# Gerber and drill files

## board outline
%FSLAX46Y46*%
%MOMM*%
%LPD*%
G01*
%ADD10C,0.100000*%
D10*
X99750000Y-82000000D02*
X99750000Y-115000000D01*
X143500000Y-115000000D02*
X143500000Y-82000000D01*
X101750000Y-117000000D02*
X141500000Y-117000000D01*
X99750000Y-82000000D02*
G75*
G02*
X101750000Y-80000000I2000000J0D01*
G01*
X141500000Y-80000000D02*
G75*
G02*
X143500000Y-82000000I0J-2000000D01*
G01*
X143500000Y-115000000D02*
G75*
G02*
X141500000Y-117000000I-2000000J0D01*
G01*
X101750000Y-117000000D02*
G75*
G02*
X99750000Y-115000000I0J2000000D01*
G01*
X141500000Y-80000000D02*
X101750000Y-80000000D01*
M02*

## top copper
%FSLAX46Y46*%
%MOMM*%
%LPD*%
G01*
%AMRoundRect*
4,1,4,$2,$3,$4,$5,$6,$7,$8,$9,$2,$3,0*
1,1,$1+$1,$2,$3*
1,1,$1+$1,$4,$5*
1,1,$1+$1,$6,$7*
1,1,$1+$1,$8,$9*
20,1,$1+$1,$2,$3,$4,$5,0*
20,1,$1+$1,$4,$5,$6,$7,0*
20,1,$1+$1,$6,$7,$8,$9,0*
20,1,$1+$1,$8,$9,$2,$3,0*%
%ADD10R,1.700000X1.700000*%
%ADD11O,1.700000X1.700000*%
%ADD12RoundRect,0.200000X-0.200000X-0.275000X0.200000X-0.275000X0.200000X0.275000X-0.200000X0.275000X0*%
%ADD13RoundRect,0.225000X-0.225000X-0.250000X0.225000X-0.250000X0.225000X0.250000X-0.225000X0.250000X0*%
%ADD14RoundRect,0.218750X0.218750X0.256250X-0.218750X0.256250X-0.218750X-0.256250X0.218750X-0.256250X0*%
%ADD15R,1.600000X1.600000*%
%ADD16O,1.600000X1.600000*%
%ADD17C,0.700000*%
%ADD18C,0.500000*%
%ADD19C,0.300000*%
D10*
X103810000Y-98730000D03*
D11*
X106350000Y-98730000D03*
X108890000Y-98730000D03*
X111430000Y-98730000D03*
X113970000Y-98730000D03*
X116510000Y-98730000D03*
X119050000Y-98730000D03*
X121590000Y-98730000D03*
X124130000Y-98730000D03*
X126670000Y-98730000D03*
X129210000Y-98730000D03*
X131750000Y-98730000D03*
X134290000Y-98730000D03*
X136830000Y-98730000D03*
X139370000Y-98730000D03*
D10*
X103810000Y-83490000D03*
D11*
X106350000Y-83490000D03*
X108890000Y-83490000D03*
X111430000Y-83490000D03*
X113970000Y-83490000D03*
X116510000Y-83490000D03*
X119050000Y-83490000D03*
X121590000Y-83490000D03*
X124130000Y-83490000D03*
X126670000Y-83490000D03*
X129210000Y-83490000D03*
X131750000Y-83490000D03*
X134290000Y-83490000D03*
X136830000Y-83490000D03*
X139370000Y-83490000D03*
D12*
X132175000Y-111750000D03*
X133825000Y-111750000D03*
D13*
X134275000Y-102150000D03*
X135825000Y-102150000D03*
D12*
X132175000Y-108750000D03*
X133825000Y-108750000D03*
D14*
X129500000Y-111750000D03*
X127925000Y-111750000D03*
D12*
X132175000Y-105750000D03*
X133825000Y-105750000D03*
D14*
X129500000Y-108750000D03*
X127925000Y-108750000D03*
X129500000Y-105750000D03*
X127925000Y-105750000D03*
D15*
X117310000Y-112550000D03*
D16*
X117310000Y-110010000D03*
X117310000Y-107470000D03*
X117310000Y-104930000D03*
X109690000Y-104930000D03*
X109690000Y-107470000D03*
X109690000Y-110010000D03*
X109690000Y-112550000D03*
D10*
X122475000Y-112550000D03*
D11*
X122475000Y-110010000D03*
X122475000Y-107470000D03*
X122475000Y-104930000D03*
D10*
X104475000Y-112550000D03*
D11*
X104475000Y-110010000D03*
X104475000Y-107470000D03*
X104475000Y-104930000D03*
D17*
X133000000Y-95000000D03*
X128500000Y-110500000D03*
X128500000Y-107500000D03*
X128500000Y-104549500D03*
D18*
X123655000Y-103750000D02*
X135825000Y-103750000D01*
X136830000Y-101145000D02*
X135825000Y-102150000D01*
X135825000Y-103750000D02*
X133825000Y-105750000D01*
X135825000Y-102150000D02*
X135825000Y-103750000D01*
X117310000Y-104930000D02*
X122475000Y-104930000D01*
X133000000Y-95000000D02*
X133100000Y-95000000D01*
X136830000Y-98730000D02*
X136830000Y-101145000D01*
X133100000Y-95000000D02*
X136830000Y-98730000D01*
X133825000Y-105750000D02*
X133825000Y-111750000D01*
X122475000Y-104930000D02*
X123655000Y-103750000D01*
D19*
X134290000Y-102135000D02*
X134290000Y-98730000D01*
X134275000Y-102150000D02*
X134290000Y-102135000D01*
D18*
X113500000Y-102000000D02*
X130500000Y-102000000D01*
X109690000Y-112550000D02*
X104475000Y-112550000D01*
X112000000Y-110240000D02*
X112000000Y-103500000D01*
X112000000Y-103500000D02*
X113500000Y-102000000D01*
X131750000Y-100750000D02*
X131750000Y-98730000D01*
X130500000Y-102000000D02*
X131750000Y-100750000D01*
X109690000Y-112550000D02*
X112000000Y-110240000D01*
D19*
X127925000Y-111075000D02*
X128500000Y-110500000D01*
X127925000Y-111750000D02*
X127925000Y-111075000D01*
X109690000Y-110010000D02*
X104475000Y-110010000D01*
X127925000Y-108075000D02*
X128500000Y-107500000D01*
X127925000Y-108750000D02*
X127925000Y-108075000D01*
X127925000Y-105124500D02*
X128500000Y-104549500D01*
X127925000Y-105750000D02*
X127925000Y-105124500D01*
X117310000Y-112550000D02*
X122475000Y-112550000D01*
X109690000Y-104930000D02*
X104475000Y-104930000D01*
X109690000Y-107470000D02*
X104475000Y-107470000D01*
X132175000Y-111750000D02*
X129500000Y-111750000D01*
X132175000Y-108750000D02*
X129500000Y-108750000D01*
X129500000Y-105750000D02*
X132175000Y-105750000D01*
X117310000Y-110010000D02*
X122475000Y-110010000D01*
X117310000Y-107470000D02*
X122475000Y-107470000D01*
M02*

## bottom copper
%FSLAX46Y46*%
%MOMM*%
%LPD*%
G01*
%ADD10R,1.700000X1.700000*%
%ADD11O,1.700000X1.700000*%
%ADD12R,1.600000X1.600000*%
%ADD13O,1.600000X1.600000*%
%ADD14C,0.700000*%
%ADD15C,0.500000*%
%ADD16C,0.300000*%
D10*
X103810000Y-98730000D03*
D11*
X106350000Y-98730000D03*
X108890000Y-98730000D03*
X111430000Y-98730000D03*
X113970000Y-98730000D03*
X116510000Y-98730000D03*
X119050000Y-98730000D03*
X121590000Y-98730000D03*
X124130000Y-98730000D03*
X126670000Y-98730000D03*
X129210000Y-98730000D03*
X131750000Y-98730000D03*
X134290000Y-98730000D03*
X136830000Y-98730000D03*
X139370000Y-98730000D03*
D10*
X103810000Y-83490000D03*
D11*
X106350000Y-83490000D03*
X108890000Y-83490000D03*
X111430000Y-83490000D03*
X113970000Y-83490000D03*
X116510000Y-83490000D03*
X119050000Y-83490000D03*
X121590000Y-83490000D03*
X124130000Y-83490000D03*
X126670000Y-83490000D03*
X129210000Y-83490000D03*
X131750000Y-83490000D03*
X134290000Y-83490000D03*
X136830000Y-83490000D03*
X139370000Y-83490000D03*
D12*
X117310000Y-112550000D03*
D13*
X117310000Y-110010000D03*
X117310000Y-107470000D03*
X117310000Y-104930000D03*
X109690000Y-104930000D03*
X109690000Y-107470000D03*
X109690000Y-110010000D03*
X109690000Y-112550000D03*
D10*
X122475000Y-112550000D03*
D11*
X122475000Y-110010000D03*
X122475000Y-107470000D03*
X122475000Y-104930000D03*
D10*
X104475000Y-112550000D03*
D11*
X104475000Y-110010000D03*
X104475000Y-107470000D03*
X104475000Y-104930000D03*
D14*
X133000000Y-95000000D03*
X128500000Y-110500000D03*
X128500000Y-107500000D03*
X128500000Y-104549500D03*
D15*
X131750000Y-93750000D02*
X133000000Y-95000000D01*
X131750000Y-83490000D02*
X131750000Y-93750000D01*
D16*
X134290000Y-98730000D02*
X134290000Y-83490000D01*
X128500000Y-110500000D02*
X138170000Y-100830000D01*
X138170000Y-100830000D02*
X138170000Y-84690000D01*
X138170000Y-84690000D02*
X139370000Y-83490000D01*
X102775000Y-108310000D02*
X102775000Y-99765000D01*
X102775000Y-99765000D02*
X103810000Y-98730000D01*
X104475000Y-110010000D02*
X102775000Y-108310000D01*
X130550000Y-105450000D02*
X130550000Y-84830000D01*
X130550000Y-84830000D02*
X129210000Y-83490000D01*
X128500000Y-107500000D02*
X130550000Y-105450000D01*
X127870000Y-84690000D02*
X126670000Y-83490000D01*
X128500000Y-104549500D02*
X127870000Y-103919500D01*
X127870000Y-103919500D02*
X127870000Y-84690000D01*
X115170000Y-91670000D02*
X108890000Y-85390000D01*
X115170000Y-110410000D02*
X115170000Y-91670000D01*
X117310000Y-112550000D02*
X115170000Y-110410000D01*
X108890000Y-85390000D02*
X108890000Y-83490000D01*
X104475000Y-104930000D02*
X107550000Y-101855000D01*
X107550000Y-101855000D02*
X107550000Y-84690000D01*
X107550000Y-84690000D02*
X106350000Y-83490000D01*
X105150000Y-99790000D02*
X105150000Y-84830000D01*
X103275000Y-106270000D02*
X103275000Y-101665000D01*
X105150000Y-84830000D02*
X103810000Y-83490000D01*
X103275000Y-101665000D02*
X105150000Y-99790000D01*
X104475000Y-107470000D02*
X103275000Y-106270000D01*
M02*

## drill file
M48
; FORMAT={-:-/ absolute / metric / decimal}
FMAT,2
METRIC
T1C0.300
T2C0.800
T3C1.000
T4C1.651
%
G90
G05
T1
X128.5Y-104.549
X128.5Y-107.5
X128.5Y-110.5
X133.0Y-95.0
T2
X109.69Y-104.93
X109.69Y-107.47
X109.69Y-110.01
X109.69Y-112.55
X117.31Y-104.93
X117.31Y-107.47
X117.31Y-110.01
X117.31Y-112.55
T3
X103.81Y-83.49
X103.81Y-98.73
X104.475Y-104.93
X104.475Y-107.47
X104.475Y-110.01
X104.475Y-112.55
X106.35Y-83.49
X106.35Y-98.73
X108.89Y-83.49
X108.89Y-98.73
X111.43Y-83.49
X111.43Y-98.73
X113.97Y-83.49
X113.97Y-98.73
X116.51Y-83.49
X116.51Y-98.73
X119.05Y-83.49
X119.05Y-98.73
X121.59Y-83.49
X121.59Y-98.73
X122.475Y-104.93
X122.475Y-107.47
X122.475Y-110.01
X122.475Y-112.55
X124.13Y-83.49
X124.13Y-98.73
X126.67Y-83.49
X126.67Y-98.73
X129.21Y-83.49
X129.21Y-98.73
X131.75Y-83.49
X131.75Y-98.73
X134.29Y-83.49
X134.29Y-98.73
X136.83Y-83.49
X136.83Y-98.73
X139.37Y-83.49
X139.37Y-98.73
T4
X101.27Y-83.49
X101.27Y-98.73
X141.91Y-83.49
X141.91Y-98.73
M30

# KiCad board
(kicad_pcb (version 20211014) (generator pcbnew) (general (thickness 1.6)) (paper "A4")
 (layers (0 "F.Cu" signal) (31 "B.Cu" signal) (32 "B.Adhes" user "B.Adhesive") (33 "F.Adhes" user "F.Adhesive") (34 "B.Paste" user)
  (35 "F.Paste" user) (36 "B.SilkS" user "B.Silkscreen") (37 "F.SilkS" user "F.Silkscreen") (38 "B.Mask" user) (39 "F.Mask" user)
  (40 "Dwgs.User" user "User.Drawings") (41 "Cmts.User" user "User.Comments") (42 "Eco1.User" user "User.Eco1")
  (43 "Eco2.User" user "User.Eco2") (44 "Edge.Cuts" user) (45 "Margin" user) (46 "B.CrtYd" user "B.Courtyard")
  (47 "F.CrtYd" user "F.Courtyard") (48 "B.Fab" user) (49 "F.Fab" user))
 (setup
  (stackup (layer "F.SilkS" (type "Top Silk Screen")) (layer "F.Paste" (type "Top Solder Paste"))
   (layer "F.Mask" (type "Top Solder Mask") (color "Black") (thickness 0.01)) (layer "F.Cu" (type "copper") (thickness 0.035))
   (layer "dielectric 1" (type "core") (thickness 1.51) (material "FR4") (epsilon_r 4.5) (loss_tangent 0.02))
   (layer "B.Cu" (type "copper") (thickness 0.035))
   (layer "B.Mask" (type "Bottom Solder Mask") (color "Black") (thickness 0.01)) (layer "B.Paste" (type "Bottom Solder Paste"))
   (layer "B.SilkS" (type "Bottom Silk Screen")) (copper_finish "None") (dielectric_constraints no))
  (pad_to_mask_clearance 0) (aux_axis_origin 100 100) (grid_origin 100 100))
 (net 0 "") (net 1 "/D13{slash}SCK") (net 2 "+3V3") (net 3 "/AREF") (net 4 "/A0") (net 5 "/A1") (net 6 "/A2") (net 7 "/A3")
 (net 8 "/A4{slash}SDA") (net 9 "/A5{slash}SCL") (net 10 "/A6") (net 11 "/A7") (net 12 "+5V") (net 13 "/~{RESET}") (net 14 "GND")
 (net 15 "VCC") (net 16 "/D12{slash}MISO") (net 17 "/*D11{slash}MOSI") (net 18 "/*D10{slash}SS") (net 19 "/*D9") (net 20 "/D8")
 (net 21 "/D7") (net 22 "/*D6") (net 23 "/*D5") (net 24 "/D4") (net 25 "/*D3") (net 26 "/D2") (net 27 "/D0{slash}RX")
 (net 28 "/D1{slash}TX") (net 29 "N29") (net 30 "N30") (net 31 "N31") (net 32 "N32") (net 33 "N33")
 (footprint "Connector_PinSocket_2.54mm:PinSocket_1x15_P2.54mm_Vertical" (layer "F.Cu") (at 103.81 98.73 90)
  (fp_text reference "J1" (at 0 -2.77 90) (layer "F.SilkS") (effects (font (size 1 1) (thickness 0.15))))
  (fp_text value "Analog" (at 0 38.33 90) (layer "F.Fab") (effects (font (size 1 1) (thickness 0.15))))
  (pad "1" thru_hole rect (at 0 0 90) (size 1.7 1.7) (drill 1) (layers *.Cu *.Mask) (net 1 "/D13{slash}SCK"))
  (pad "2" thru_hole oval (at 0 2.54 90) (size 1.7 1.7) (drill 1) (layers *.Cu *.Mask) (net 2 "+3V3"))
  (pad "3" thru_hole oval (at 0 5.08 90) (size 1.7 1.7) (drill 1) (layers *.Cu *.Mask) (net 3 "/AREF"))
  (pad "4" thru_hole oval (at 0 7.62 90) (size 1.7 1.7) (drill 1) (layers *.Cu *.Mask) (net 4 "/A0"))
  (pad "5" thru_hole oval (at 0 10.16 90) (size 1.7 1.7) (drill 1) (layers *.Cu *.Mask) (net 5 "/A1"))
  (pad "6" thru_hole oval (at 0 12.7 90) (size 1.7 1.7) (drill 1) (layers *.Cu *.Mask) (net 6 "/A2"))
  (pad "7" thru_hole oval (at 0 15.24 90) (size 1.7 1.7) (drill 1) (layers *.Cu *.Mask) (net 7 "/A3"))
  (pad "8" thru_hole oval (at 0 17.78 90) (size 1.7 1.7) (drill 1) (layers *.Cu *.Mask) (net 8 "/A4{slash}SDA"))
  (pad "9" thru_hole oval (at 0 20.32 90) (size 1.7 1.7) (drill 1) (layers *.Cu *.Mask) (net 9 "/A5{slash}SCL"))
  (pad "10" thru_hole oval (at 0 22.86 90) (size 1.7 1.7) (drill 1) (layers *.Cu *.Mask) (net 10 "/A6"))
  (pad "11" thru_hole oval (at 0 25.4 90) (size 1.7 1.7) (drill 1) (layers *.Cu *.Mask) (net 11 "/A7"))
  (pad "12" thru_hole oval (at 0 27.94 90) (size 1.7 1.7) (drill 1) (layers *.Cu *.Mask) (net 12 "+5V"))
  (pad "13" thru_hole oval (at 0 30.48 90) (size 1.7 1.7) (drill 1) (layers *.Cu *.Mask) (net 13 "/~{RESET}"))
  (pad "14" thru_hole oval (at 0 33.02 90) (size 1.7 1.7) (drill 1) (layers *.Cu *.Mask) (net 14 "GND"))
  (pad "15" thru_hole oval (at 0 35.56 90) (size 1.7 1.7) (drill 1) (layers *.Cu *.Mask) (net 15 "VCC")))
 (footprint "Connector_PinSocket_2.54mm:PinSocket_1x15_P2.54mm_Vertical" (layer "F.Cu") (at 103.81 83.49 90)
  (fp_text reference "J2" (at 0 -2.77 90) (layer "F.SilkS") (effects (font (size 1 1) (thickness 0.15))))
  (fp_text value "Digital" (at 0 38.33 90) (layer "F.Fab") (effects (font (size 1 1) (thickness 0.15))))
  (pad "1" thru_hole rect (at 0 0 90) (size 1.7 1.7) (drill 1) (layers *.Cu *.Mask) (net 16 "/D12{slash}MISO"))
  (pad "2" thru_hole oval (at 0 2.54 90) (size 1.7 1.7) (drill 1) (layers *.Cu *.Mask) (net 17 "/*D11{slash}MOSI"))
  (pad "3" thru_hole oval (at 0 5.08 90) (size 1.7 1.7) (drill 1) (layers *.Cu *.Mask) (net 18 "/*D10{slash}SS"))
  (pad "4" thru_hole oval (at 0 7.62 90) (size 1.7 1.7) (drill 1) (layers *.Cu *.Mask) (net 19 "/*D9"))
  (pad "5" thru_hole oval (at 0 10.16 90) (size 1.7 1.7) (drill 1) (layers *.Cu *.Mask) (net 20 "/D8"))
  (pad "6" thru_hole oval (at 0 12.7 90) (size 1.7 1.7) (drill 1) (layers *.Cu *.Mask) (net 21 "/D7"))
  (pad "7" thru_hole oval (at 0 15.24 90) (size 1.7 1.7) (drill 1) (layers *.Cu *.Mask) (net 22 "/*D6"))
  (pad "8" thru_hole oval (at 0 17.78 90) (size 1.7 1.7) (drill 1) (layers *.Cu *.Mask) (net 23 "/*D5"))
  (pad "9" thru_hole oval (at 0 20.32 90) (size 1.7 1.7) (drill 1) (layers *.Cu *.Mask) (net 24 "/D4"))
  (pad "10" thru_hole oval (at 0 22.86 90) (size 1.7 1.7) (drill 1) (layers *.Cu *.Mask) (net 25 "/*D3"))
  (pad "11" thru_hole oval (at 0 25.4 90) (size 1.7 1.7) (drill 1) (layers *.Cu *.Mask) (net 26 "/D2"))
  (pad "12" thru_hole oval (at 0 27.94 90) (size 1.7 1.7) (drill 1) (layers *.Cu *.Mask) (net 14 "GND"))
  (pad "13" thru_hole oval (at 0 30.48 90) (size 1.7 1.7) (drill 1) (layers *.Cu *.Mask) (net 13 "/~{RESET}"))
  (pad "14" thru_hole oval (at 0 33.02 90) (size 1.7 1.7) (drill 1) (layers *.Cu *.Mask) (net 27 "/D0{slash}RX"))
  (pad "15" thru_hole oval (at 0 35.56 90) (size 1.7 1.7) (drill 1) (layers *.Cu *.Mask) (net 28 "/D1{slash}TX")))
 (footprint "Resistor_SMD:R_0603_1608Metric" (layer "F.Cu") (at 133 111.75)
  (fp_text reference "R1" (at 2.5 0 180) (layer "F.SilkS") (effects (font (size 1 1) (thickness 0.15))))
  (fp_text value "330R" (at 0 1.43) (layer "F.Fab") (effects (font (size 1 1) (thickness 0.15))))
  (pad "1" smd roundrect (at -0.825 0) (size 0.8 0.95) (layers "F.Cu" "F.Paste" "F.Mask") (roundrect_rratio 0.25) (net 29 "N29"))
  (pad "2" smd roundrect (at 0.825 0) (size 0.8 0.95) (layers "F.Cu" "F.Paste" "F.Mask") (roundrect_rratio 0.25) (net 14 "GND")))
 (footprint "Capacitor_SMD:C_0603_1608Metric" (layer "F.Cu") (at 135.05 102.15)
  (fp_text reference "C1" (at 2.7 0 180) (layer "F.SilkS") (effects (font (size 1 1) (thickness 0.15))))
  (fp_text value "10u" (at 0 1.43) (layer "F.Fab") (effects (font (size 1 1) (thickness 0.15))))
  (pad "1" smd roundrect (at -0.775 0) (size 0.9 0.95) (layers "F.Cu" "F.Paste" "F.Mask") (roundrect_rratio 0.25) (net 13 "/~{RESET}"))
  (pad "2" smd roundrect (at 0.775 0) (size 0.9 0.95) (layers "F.Cu" "F.Paste" "F.Mask") (roundrect_rratio 0.25) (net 14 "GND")))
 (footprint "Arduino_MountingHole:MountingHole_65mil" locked (layer "F.Cu") (at 101.27 83.49)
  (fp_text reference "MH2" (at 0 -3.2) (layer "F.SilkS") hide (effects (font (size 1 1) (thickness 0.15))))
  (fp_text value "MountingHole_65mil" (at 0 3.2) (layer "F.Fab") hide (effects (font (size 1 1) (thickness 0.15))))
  (pad "" np_thru_hole circle locked (at 0 0) (size 1.651 1.651) (drill 1.651) (layers F&B.Cu *.Mask)))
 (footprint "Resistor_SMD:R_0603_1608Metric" (layer "F.Cu") (at 133 108.75)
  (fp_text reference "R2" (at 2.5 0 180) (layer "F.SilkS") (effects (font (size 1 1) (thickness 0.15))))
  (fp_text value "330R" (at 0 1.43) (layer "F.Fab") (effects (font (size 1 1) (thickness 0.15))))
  (pad "1" smd roundrect (at -0.825 0) (size 0.8 0.95) (layers "F.Cu" "F.Paste" "F.Mask") (roundrect_rratio 0.25) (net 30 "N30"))
  (pad "2" smd roundrect (at 0.825 0) (size 0.8 0.95) (layers "F.Cu" "F.Paste" "F.Mask") (roundrect_rratio 0.25) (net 14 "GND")))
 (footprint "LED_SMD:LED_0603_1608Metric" (layer "F.Cu") (at 128.7125 111.75 180)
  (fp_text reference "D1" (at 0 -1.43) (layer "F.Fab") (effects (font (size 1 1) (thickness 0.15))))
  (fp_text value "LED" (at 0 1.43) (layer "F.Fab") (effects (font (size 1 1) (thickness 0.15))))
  (pad "1" smd roundrect (at -0.7875 0 180) (size 0.875 0.95) (layers "F.Cu" "F.Paste" "F.Mask") (roundrect_rratio 0.25) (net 29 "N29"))
  (pad "2" smd roundrect (at 0.7875 0 180) (size 0.875 0.95) (layers "F.Cu" "F.Paste" "F.Mask") (roundrect_rratio 0.25)
   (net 28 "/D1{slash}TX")))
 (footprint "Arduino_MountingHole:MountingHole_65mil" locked (layer "F.Cu") (at 141.91 98.73)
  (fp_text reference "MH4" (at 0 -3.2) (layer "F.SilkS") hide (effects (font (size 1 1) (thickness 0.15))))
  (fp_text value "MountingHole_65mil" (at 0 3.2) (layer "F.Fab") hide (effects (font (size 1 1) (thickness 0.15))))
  (pad "" np_thru_hole circle locked (at 0 0) (size 1.651 1.651) (drill 1.651) (layers F&B.Cu *.Mask)))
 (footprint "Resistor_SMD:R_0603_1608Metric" (layer "F.Cu") (at 133 105.75)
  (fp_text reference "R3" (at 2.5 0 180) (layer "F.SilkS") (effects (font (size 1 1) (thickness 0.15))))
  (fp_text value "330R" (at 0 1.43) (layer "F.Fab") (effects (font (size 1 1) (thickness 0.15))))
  (pad "1" smd roundrect (at -0.825 0) (size 0.8 0.95) (layers "F.Cu" "F.Paste" "F.Mask") (roundrect_rratio 0.25) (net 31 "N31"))
  (pad "2" smd roundrect (at 0.825 0) (size 0.8 0.95) (layers "F.Cu" "F.Paste" "F.Mask") (roundrect_rratio 0.25) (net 14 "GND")))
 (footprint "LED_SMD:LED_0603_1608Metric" (layer "F.Cu") (at 128.7125 108.75 180)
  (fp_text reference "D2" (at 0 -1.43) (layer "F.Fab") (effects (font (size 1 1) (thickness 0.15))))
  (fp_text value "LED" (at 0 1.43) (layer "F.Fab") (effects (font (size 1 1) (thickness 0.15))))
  (pad "1" smd roundrect (at -0.7875 0 180) (size 0.875 0.95) (layers "F.Cu" "F.Paste" "F.Mask") (roundrect_rratio 0.25) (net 30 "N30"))
  (pad "2" smd roundrect (at 0.7875 0 180) (size 0.875 0.95) (layers "F.Cu" "F.Paste" "F.Mask") (roundrect_rratio 0.25) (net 26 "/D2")))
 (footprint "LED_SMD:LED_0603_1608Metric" (layer "F.Cu") (at 128.7125 105.75 180)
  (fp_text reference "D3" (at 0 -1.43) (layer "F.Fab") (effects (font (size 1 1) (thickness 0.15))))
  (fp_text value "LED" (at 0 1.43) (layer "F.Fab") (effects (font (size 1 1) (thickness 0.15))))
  (pad "1" smd roundrect (at -0.7875 0 180) (size 0.875 0.95) (layers "F.Cu" "F.Paste" "F.Mask") (roundrect_rratio 0.25) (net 31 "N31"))
  (pad "2" smd roundrect (at 0.7875 0 180) (size 0.875 0.95) (layers "F.Cu" "F.Paste" "F.Mask") (roundrect_rratio 0.25) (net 25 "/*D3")))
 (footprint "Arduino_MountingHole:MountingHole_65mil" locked (layer "F.Cu") (at 101.27 98.73)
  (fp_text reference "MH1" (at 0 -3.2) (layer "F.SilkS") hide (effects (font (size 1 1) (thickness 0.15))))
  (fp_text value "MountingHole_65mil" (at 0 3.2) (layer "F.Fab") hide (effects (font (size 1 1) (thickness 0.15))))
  (pad "" np_thru_hole circle locked (at 0 0) (size 1.651 1.651) (drill 1.651) (layers F&B.Cu *.Mask)))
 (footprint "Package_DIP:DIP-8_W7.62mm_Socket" (layer "F.Cu") (at 117.31 112.55 180)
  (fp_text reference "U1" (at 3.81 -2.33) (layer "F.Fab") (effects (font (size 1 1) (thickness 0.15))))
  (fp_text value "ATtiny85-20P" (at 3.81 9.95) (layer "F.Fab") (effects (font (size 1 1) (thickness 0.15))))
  (pad "1" thru_hole rect (at 0 0 180) (size 1.6 1.6) (drill 0.8) (layers *.Cu *.Mask) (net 18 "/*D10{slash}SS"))
  (pad "2" thru_hole oval (at 0 2.54 180) (size 1.6 1.6) (drill 0.8) (layers *.Cu *.Mask) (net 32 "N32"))
  (pad "3" thru_hole oval (at 0 5.08 180) (size 1.6 1.6) (drill 0.8) (layers *.Cu *.Mask) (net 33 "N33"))
  (pad "4" thru_hole oval (at 0 7.62 180) (size 1.6 1.6) (drill 0.8) (layers *.Cu *.Mask) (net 14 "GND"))
  (pad "5" thru_hole oval (at 7.62 7.62 180) (size 1.6 1.6) (drill 0.8) (layers *.Cu *.Mask) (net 17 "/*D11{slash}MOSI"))
  (pad "6" thru_hole oval (at 7.62 5.08 180) (size 1.6 1.6) (drill 0.8) (layers *.Cu *.Mask) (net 16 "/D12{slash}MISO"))
  (pad "7" thru_hole oval (at 7.62 2.54 180) (size 1.6 1.6) (drill 0.8) (layers *.Cu *.Mask) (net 1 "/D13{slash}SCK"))
  (pad "8" thru_hole oval (at 7.62 0 180) (size 1.6 1.6) (drill 0.8) (layers *.Cu *.Mask) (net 12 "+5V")))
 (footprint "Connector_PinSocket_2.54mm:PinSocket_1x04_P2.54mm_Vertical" (layer "F.Cu") (at 122.475 112.55 180)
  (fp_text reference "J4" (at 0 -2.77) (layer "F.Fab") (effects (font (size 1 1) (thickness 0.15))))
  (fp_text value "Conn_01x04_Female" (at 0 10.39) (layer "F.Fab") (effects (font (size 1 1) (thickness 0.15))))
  (pad "1" thru_hole rect (at 0 0 180) (size 1.7 1.7) (drill 1) (layers *.Cu *.Mask) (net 18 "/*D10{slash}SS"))
  (pad "2" thru_hole oval (at 0 2.54 180) (size 1.7 1.7) (drill 1) (layers *.Cu *.Mask) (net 32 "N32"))
  (pad "3" thru_hole oval (at 0 5.08 180) (size 1.7 1.7) (drill 1) (layers *.Cu *.Mask) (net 33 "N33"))
  (pad "4" thru_hole oval (at 0 7.62 180) (size 1.7 1.7) (drill 1) (layers *.Cu *.Mask) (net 14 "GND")))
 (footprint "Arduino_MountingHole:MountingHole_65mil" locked (layer "F.Cu") (at 141.91 83.49)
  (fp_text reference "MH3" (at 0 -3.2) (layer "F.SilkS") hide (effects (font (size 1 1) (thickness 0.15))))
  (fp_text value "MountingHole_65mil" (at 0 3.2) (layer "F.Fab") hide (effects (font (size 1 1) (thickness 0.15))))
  (pad "" np_thru_hole circle locked (at 0 0) (size 1.651 1.651) (drill 1.651) (layers F&B.Cu *.Mask)))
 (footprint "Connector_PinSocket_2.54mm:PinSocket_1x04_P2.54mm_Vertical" (layer "F.Cu") (at 104.475 112.55 180)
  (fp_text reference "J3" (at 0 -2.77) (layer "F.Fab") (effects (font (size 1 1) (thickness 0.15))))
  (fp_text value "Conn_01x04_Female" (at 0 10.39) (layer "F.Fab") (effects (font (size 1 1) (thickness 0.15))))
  (pad "1" thru_hole rect (at 0 0 180) (size 1.7 1.7) (drill 1) (layers *.Cu *.Mask) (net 12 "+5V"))
  (pad "2" thru_hole oval (at 0 2.54 180) (size 1.7 1.7) (drill 1) (layers *.Cu *.Mask) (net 1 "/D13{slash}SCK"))
  (pad "3" thru_hole oval (at 0 5.08 180) (size 1.7 1.7) (drill 1) (layers *.Cu *.Mask) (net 16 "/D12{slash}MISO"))
  (pad "4" thru_hole oval (at 0 7.62 180) (size 1.7 1.7) (drill 1) (layers *.Cu *.Mask) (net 17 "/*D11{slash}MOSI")))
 (gr_line (start 99.75 82) (end 99.75 115) (layer "Edge.Cuts") (width 0.1))
 (gr_line (start 143.5 115) (end 143.5 82) (layer "Edge.Cuts") (width 0.1))
 (gr_line (start 101.75 117) (end 141.5 117) (layer "Edge.Cuts") (width 0.1))
 (gr_arc (start 99.75 82) (mid 100.335786 80.585786) (end 101.75 80) (layer "Edge.Cuts") (width 0.1))
 (gr_arc (start 141.5 80) (mid 142.914214 80.585786) (end 143.5 82) (layer "Edge.Cuts") (width 0.1))
 (gr_arc (start 143.5 115) (mid 142.914214 116.414214) (end 141.5 117) (layer "Edge.Cuts") (width 0.1))
 (gr_arc (start 101.75 117) (mid 100.335786 116.414214) (end 99.75 115) (layer "Edge.Cuts") (width 0.1))
 (gr_line (start 141.5 80) (end 101.75 80) (layer "Edge.Cuts") (width 0.1))
 (segment (start 123.655 103.75) (end 135.825 103.75) (width 0.5) (layer "F.Cu") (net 14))
 (segment (start 136.83 101.145) (end 135.825 102.15) (width 0.5) (layer "F.Cu") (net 14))
 (segment (start 135.825 103.75) (end 133.825 105.75) (width 0.5) (layer "F.Cu") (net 14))
 (segment (start 135.825 102.15) (end 135.825 103.75) (width 0.5) (layer "F.Cu") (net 14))
 (segment (start 117.31 104.93) (end 122.475 104.93) (width 0.5) (layer "F.Cu") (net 14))
 (segment (start 133 95) (end 133.1 95) (width 0.5) (layer "F.Cu") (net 14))
 (segment (start 136.83 98.73) (end 136.83 101.145) (width 0.5) (layer "F.Cu") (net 14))
 (segment (start 133.1 95) (end 136.83 98.73) (width 0.5) (layer "F.Cu") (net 14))
 (segment (start 133.825 105.75) (end 133.825 111.75) (width 0.5) (layer "F.Cu") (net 14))
 (segment (start 122.475 104.93) (end 123.655 103.75) (width 0.5) (layer "F.Cu") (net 14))
 (via (at 133 95) (size 0.7) (drill 0.3) (layers "F.Cu" "B.Cu") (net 14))
 (segment (start 131.75 93.75) (end 133 95) (width 0.5) (layer "B.Cu") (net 14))
 (segment (start 131.75 83.49) (end 131.75 93.75) (width 0.5) (layer "B.Cu") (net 14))
 (segment (start 134.29 102.135) (end 134.29 98.73) (width 0.3) (layer "F.Cu") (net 13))
 (segment (start 134.275 102.15) (end 134.29 102.135) (width 0.3) (layer "F.Cu") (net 13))
 (segment (start 134.29 98.73) (end 134.29 83.49) (width 0.3) (layer "B.Cu") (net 13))
 (segment (start 113.5 102) (end 130.5 102) (width 0.5) (layer "F.Cu") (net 12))
 (segment (start 109.69 112.55) (end 104.475 112.55) (width 0.5) (layer "F.Cu") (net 12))
 (segment (start 112 110.24) (end 112 103.5) (width 0.5) (layer "F.Cu") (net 12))
 (segment (start 112 103.5) (end 113.5 102) (width 0.5) (layer "F.Cu") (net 12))
 (segment (start 131.75 100.75) (end 131.75 98.73) (width 0.5) (layer "F.Cu") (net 12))
 (segment (start 130.5 102) (end 131.75 100.75) (width 0.5) (layer "F.Cu") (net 12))
 (segment (start 109.69 112.55) (end 112 110.24) (width 0.5) (layer "F.Cu") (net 12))
 (segment (start 127.925 111.075) (end 128.5 110.5) (width 0.3) (layer "F.Cu") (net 28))
 (segment (start 127.925 111.75) (end 127.925 111.075) (width 0.3) (layer "F.Cu") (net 28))
 (via (at 128.5 110.5) (size 0.7) (drill 0.3) (layers "F.Cu" "B.Cu") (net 28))
 (segment (start 128.5 110.5) (end 138.17 100.83) (width 0.3) (layer "B.Cu") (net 28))
 (segment (start 138.17 100.83) (end 138.17 84.69) (width 0.3) (layer "B.Cu") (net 28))
 (segment (start 138.17 84.69) (end 139.37 83.49) (width 0.3) (layer "B.Cu") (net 28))
 (segment (start 109.69 110.01) (end 104.475 110.01) (width 0.3) (layer "F.Cu") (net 1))
 (segment (start 102.775 108.31) (end 102.775 99.765) (width 0.3) (layer "B.Cu") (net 1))
 (segment (start 102.775 99.765) (end 103.81 98.73) (width 0.3) (layer "B.Cu") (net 1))
 (segment (start 104.475 110.01) (end 102.775 108.31) (width 0.3) (layer "B.Cu") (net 1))
 (segment (start 127.925 108.075) (end 128.5 107.5) (width 0.3) (layer "F.Cu") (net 26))
 (segment (start 127.925 108.75) (end 127.925 108.075) (width 0.3) (layer "F.Cu") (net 26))
 (via (at 128.5 107.5) (size 0.7) (drill 0.3) (layers "F.Cu" "B.Cu") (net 26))
 (segment (start 130.55 105.45) (end 130.55 84.83) (width 0.3) (layer "B.Cu") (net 26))
 (segment (start 130.55 84.83) (end 129.21 83.49) (width 0.3) (layer "B.Cu") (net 26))
 (segment (start 128.5 107.5) (end 130.55 105.45) (width 0.3) (layer "B.Cu") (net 26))
 (segment (start 127.925 105.1245) (end 128.5 104.5495) (width 0.3) (layer "F.Cu") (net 25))
 (segment (start 127.925 105.75) (end 127.925 105.1245) (width 0.3) (layer "F.Cu") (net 25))
 (via (at 128.5 104.5495) (size 0.7) (drill 0.3) (layers "F.Cu" "B.Cu") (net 25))
 (segment (start 127.87 84.69) (end 126.67 83.49) (width 0.3) (layer "B.Cu") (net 25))
 (segment (start 128.5 104.5495) (end 127.87 103.9195) (width 0.3) (layer "B.Cu") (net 25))
 (segment (start 127.87 103.9195) (end 127.87 84.69) (width 0.3) (layer "B.Cu") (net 25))
 (segment (start 117.31 112.55) (end 122.475 112.55) (width 0.3) (layer "F.Cu") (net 18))
 (segment (start 115.17 91.67) (end 108.89 85.39) (width 0.3) (layer "B.Cu") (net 18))
 (segment (start 115.17 110.41) (end 115.17 91.67) (width 0.3) (layer "B.Cu") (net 18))
 (segment (start 117.31 112.55) (end 115.17 110.41) (width 0.3) (layer "B.Cu") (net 18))
 (segment (start 108.89 85.39) (end 108.89 83.49) (width 0.3) (layer "B.Cu") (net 18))
 (segment (start 109.69 104.93) (end 104.475 104.93) (width 0.3) (layer "F.Cu") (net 17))
 (segment (start 104.475 104.93) (end 107.55 101.855) (width 0.3) (layer "B.Cu") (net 17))
 (segment (start 107.55 101.855) (end 107.55 84.69) (width 0.3) (layer "B.Cu") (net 17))
 (segment (start 107.55 84.69) (end 106.35 83.49) (width 0.3) (layer "B.Cu") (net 17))
 (segment (start 109.69 107.47) (end 104.475 107.47) (width 0.3) (layer "F.Cu") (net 16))
 (segment (start 105.15 99.79) (end 105.15 84.83) (width 0.3) (layer "B.Cu") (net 16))
 (segment (start 103.275 106.27) (end 103.275 101.665) (width 0.3) (layer "B.Cu") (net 16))
 (segment (start 105.15 84.83) (end 103.81 83.49) (width 0.3) (layer "B.Cu") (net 16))
 (segment (start 103.275 101.665) (end 105.15 99.79) (width 0.3) (layer "B.Cu") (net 16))
 (segment (start 104.475 107.47) (end 103.275 106.27) (width 0.3) (layer "B.Cu") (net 16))
 (segment (start 132.175 111.75) (end 129.5 111.75) (width 0.3) (layer "F.Cu") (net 29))
 (segment (start 132.175 108.75) (end 129.5 108.75) (width 0.3) (layer "F.Cu") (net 30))
 (segment (start 129.5 105.75) (end 132.175 105.75) (width 0.3) (layer "F.Cu") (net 31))
 (segment (start 117.31 110.01) (end 122.475 110.01) (width 0.3) (layer "F.Cu") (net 32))
 (segment (start 117.31 107.47) (end 122.475 107.47) (width 0.3) (layer "F.Cu") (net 33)))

